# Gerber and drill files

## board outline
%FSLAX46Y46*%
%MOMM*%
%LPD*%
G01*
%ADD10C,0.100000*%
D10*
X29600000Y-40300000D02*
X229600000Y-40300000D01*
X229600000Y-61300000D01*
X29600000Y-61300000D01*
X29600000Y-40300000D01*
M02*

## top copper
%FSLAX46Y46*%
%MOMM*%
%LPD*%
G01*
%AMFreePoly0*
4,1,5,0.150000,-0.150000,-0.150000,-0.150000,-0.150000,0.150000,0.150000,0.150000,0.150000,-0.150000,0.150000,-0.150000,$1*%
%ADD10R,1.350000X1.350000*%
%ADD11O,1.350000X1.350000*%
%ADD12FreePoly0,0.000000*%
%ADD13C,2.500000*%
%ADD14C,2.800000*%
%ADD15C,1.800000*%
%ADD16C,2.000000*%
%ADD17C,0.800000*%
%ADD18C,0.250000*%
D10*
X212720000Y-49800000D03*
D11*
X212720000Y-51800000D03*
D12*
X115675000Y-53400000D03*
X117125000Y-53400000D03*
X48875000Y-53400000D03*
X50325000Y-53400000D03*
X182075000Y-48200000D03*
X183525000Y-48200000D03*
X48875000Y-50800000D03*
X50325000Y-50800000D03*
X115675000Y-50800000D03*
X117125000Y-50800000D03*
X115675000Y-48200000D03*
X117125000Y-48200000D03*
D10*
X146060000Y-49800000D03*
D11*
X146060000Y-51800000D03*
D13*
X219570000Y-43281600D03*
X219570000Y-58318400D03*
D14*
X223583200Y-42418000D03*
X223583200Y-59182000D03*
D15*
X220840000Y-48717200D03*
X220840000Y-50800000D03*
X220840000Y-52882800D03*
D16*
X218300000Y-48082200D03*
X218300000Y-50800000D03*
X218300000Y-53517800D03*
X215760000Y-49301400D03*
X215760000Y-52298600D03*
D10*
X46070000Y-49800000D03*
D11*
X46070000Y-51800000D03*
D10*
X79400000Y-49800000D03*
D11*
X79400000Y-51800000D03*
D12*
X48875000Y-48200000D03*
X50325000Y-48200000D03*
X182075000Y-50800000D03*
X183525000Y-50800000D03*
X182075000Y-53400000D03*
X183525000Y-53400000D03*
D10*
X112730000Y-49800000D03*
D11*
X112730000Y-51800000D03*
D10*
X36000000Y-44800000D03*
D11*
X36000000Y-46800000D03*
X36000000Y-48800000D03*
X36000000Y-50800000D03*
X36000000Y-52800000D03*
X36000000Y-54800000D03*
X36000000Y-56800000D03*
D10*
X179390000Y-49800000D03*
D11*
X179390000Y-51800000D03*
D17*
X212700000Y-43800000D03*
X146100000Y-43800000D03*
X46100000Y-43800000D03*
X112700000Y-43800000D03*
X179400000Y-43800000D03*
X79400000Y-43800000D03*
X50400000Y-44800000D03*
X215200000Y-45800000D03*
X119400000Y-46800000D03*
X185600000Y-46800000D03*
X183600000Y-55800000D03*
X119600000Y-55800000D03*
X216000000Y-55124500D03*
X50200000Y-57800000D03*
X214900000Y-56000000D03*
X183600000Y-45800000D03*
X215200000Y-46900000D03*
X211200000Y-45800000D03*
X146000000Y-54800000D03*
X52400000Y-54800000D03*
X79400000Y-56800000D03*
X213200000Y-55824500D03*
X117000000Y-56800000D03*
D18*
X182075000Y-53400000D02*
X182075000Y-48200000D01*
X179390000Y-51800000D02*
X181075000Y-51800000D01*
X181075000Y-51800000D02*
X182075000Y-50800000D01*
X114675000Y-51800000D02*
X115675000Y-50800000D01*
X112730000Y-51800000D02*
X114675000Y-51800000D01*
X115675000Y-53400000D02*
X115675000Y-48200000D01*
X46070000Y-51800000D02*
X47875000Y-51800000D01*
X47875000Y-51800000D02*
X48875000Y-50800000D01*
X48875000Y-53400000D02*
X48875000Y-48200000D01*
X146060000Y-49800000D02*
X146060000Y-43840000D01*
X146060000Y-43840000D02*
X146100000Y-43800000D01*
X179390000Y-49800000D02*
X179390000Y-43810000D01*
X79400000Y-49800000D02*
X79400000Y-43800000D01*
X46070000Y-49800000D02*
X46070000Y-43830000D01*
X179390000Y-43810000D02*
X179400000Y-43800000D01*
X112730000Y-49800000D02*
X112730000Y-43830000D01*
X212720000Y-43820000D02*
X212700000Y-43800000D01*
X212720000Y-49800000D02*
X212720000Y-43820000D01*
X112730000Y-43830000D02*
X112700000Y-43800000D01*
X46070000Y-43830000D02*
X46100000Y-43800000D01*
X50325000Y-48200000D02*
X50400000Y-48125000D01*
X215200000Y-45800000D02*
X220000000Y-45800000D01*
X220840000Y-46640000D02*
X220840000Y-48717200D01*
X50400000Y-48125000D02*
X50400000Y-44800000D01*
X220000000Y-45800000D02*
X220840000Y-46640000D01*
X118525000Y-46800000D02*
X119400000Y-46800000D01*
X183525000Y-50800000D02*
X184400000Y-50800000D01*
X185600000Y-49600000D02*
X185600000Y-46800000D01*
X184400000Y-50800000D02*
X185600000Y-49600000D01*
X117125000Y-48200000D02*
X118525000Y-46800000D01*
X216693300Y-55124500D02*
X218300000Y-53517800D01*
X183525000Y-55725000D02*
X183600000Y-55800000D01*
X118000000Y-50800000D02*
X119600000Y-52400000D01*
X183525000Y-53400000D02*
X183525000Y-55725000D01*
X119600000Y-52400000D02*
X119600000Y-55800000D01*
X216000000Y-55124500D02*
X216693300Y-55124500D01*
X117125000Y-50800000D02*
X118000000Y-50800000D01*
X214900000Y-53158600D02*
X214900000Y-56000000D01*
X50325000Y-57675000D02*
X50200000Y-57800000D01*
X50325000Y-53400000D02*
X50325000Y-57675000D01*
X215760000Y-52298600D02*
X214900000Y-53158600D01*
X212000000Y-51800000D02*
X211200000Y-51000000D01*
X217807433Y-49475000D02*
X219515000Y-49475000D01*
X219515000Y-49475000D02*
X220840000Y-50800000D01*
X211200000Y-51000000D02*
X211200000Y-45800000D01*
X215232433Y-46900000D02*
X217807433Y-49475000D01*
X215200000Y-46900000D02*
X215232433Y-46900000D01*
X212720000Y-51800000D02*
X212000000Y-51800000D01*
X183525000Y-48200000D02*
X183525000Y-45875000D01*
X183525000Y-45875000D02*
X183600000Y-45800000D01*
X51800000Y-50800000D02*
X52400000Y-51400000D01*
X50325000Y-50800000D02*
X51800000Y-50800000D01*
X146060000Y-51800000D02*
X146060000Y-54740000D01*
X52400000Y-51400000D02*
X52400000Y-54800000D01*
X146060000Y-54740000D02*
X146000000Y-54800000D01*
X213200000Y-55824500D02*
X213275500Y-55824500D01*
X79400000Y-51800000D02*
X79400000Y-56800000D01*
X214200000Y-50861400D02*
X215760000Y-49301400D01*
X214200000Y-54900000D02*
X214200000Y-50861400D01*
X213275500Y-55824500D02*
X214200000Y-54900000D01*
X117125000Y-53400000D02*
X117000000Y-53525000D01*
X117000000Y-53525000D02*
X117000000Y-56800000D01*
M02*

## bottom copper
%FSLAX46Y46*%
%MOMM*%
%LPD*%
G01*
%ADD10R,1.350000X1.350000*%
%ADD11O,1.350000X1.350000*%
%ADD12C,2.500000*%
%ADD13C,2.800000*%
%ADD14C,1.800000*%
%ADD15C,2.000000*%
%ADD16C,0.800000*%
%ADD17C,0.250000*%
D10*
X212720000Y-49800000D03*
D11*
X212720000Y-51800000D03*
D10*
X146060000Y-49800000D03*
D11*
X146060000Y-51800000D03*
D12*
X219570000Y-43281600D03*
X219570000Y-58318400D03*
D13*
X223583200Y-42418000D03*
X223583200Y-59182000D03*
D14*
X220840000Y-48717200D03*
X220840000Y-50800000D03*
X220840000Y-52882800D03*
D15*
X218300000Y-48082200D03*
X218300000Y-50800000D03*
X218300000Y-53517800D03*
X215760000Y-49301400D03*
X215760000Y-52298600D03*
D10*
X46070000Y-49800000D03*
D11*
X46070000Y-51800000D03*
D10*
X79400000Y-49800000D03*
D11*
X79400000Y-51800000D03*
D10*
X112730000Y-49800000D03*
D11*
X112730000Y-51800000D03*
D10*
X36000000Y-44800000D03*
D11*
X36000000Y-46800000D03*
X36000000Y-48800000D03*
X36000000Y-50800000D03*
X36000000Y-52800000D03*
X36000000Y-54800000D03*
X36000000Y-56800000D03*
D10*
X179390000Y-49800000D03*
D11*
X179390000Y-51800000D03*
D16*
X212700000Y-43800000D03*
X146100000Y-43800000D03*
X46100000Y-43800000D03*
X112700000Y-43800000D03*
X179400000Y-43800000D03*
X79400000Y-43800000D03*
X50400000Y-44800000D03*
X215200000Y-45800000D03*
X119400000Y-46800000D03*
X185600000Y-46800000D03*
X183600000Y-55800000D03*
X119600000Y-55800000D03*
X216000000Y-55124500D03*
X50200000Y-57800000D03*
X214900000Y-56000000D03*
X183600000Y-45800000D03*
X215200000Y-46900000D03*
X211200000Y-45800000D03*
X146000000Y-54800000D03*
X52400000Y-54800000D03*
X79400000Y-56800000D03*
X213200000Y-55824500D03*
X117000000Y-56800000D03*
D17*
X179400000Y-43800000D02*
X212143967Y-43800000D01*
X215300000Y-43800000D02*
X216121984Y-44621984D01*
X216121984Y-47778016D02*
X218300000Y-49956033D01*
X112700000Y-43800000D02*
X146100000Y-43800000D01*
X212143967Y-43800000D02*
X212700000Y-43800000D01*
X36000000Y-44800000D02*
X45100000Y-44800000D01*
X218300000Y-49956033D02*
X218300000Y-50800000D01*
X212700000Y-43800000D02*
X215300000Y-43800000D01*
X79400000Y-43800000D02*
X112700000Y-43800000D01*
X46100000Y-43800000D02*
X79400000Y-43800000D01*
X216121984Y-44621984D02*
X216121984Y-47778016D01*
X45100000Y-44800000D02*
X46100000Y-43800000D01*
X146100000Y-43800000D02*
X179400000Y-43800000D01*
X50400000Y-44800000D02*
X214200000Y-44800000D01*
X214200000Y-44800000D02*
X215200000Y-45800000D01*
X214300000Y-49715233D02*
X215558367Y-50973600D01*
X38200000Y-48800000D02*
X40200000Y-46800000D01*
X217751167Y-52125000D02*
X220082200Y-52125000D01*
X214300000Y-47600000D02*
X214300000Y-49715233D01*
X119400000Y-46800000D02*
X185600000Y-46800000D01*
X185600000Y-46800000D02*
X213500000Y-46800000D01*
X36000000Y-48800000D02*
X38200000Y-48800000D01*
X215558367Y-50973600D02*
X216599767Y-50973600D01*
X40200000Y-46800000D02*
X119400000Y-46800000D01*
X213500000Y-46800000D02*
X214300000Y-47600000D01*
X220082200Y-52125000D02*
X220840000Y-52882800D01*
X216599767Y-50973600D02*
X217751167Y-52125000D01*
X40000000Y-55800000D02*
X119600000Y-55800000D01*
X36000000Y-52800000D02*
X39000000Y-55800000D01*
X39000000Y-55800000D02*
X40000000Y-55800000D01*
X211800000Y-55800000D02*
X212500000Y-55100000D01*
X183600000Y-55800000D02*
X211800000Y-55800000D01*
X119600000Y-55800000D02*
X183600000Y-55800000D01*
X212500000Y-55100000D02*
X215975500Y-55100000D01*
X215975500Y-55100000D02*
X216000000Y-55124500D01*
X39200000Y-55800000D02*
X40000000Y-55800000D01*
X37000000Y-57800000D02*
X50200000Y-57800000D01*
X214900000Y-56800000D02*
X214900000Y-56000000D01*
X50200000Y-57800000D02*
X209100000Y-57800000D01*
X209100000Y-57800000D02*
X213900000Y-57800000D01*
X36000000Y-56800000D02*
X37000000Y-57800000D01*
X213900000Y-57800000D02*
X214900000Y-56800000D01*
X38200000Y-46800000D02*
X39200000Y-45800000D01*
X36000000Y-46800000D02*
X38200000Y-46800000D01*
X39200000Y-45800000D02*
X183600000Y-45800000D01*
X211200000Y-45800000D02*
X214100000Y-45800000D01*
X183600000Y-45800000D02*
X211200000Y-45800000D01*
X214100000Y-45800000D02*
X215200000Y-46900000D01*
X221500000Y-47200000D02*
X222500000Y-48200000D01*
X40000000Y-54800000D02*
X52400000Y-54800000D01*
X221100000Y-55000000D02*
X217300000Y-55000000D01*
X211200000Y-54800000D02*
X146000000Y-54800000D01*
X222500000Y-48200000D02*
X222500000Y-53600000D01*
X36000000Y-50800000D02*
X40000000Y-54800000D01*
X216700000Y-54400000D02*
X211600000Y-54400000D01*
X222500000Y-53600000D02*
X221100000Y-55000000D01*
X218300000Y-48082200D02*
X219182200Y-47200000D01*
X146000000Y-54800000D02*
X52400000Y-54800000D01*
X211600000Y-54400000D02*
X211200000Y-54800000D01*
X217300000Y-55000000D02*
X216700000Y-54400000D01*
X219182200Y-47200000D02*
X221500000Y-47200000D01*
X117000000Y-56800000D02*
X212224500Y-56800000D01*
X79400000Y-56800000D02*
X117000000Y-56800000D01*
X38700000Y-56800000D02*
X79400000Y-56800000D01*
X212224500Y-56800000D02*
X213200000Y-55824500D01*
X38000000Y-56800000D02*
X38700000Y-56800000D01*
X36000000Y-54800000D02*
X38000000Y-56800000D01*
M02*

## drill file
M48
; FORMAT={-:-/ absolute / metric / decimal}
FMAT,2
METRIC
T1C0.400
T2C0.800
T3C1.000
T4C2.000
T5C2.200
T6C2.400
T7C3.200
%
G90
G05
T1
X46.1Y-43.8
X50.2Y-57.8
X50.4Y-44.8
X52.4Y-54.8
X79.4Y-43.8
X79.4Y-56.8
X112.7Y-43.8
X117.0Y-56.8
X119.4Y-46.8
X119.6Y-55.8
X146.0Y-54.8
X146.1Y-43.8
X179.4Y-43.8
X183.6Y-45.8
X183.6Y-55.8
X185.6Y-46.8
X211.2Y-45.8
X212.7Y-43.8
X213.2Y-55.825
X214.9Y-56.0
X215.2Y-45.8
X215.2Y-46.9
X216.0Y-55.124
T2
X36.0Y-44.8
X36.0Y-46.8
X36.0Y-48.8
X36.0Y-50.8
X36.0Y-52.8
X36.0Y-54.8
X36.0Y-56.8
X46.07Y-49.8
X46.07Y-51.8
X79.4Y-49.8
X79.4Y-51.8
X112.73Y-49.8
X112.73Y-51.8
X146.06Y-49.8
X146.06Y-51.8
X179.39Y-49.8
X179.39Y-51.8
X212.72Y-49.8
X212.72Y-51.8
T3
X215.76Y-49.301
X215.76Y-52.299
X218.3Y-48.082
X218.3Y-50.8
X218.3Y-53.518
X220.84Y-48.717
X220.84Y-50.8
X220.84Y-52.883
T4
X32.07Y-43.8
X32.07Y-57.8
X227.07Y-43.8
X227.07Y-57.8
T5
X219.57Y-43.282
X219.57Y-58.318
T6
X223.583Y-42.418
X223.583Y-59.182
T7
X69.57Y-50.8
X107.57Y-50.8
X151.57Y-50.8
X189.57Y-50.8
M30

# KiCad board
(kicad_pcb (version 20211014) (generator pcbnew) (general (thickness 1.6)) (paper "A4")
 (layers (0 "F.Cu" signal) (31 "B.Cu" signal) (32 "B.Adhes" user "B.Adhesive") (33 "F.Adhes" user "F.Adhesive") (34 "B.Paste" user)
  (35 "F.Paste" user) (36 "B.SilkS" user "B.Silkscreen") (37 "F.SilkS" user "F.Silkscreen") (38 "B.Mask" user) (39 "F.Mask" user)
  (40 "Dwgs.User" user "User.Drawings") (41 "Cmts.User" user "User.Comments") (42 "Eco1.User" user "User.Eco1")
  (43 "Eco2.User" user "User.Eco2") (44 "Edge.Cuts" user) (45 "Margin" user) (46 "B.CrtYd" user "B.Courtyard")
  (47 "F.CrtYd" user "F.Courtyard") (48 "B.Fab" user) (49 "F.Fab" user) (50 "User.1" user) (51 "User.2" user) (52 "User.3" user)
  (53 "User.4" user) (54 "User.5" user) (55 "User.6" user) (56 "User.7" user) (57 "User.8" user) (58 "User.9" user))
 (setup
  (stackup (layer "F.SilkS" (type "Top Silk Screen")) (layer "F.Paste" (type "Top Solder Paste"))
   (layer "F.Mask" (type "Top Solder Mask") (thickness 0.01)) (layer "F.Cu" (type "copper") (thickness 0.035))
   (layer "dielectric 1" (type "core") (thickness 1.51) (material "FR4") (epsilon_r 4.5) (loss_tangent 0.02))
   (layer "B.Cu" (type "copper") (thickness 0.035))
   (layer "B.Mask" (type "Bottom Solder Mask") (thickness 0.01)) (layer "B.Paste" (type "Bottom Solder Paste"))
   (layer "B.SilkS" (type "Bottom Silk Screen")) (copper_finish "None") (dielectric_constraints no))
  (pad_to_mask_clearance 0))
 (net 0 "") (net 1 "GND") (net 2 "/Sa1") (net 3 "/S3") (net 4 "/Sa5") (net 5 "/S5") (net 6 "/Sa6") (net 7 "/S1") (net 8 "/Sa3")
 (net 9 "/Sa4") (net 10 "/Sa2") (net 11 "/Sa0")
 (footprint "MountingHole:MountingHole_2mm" (layer "F.Cu") (at 32.07 57.8)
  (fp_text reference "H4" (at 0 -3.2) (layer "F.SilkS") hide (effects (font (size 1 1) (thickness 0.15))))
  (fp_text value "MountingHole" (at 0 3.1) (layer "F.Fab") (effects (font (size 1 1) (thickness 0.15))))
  (pad "" np_thru_hole circle (at 0 0) (size 2 2) (drill 2) (layers *.Cu *.Mask)))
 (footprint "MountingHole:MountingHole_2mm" (layer "F.Cu") (at 227.07 57.8)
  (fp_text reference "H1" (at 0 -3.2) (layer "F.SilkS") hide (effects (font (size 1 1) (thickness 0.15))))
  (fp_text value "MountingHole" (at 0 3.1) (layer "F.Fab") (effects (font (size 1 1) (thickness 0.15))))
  (pad "" np_thru_hole circle (at 0 0) (size 2 2) (drill 2) (layers *.Cu *.Mask)))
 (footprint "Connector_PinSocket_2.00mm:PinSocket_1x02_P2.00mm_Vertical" (layer "F.Cu") (at 212.72 49.8)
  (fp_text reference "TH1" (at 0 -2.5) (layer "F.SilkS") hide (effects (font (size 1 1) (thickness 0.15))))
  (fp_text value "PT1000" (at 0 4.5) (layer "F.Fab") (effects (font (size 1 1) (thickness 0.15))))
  (pad "1" thru_hole rect (at 0 0) (size 1.35 1.35) (drill 0.8) (layers *.Cu *.Mask) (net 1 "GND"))
  (pad "2" thru_hole oval (at 0 2) (size 1.35 1.35) (drill 0.8) (layers *.Cu *.Mask) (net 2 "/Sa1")))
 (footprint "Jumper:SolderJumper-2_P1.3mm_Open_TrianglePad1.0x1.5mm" (layer "F.Cu") (at 116.4 53.4)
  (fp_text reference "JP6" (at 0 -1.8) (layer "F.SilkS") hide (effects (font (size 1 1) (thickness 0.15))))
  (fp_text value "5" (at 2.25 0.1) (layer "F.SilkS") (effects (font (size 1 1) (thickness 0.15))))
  (pad "1" smd custom (at -0.725 0) (size 0.3 0.3) (layers "F.Cu" "F.Mask") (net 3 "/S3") (zone_connect 2)
   (options (clearance outline) (anchor rect)) (primitives))
  (pad "2" smd custom (at 0.725 0) (size 0.3 0.3) (layers "F.Cu" "F.Mask") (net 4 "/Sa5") (zone_connect 2)
   (options (clearance outline) (anchor rect)) (primitives)))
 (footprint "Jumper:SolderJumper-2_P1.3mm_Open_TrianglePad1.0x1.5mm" (layer "F.Cu") (at 49.6 53.4)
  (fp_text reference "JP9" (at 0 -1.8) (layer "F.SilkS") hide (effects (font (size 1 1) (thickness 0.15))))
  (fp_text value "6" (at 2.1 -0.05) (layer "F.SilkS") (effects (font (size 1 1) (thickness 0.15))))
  (pad "1" smd custom (at -0.725 0) (size 0.3 0.3) (layers "F.Cu" "F.Mask") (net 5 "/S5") (zone_connect 2)
   (options (clearance outline) (anchor rect)) (primitives))
  (pad "2" smd custom (at 0.725 0) (size 0.3 0.3) (layers "F.Cu" "F.Mask") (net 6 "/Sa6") (zone_connect 2)
   (options (clearance outline) (anchor rect)) (primitives)))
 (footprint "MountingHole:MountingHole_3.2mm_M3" (layer "F.Cu") (at 69.57 50.8)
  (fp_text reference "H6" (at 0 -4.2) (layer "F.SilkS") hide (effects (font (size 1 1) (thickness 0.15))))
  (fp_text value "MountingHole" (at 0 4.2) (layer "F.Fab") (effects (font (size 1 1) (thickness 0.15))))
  (pad "" np_thru_hole circle (at 0 0) (size 3.2 3.2) (drill 3.2) (layers *.Cu *.Mask)))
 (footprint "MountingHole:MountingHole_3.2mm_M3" (layer "F.Cu") (at 107.57 50.8)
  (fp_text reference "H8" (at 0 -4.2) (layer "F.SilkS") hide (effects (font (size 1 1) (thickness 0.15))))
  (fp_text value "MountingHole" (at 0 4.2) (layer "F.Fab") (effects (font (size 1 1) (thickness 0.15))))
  (pad "" np_thru_hole circle (at 0 0) (size 3.2 3.2) (drill 3.2) (layers *.Cu *.Mask)))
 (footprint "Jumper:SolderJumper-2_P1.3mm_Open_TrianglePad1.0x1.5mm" (layer "F.Cu") (at 182.8 48.2)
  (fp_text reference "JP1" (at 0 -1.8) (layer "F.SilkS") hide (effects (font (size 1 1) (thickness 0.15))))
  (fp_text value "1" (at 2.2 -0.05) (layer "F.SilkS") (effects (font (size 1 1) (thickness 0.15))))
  (pad "1" smd custom (at -0.725 0) (size 0.3 0.3) (layers "F.Cu" "F.Mask") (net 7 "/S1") (zone_connect 2)
   (options (clearance outline) (anchor rect)) (primitives))
  (pad "2" smd custom (at 0.725 0) (size 0.3 0.3) (layers "F.Cu" "F.Mask") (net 2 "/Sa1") (zone_connect 2)
   (options (clearance outline) (anchor rect)) (primitives)))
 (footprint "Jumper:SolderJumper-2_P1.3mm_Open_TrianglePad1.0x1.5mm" (layer "F.Cu") (at 49.6 50.8)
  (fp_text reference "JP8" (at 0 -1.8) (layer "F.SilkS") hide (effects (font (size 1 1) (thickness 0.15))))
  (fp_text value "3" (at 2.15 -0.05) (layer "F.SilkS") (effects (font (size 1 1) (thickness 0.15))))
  (pad "1" smd custom (at -0.725 0) (size 0.3 0.3) (layers "F.Cu" "F.Mask") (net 5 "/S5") (zone_connect 2)
   (options (clearance outline) (anchor rect)) (primitives))
  (pad "2" smd custom (at 0.725 0) (size 0.3 0.3) (layers "F.Cu" "F.Mask") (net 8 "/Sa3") (zone_connect 2)
   (options (clearance outline) (anchor rect)) (primitives)))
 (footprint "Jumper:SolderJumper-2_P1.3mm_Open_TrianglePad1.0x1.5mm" (layer "F.Cu") (at 116.4 50.8)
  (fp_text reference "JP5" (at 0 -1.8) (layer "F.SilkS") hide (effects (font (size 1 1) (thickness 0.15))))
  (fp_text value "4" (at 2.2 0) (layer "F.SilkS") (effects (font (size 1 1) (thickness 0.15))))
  (pad "1" smd custom (at -0.725 0) (size 0.3 0.3) (layers "F.Cu" "F.Mask") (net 3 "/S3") (zone_connect 2)
   (options (clearance outline) (anchor rect)) (primitives))
  (pad "2" smd custom (at 0.725 0) (size 0.3 0.3) (layers "F.Cu" "F.Mask") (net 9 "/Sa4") (zone_connect 2)
   (options (clearance outline) (anchor rect)) (primitives)))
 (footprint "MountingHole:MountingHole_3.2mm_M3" (layer "F.Cu") (at 151.57 50.8)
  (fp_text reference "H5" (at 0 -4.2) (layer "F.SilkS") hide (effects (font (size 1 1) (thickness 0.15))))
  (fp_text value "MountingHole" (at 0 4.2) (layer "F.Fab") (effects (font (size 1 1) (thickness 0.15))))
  (pad "" np_thru_hole circle (at 0 0) (size 3.2 3.2) (drill 3.2) (layers *.Cu *.Mask)))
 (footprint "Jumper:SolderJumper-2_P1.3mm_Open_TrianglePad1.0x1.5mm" (layer "F.Cu") (at 116.4 48.2)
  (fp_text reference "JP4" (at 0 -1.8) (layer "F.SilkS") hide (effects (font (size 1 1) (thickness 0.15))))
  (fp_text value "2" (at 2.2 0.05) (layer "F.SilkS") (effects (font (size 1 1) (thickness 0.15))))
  (pad "1" smd custom (at -0.725 0) (size 0.3 0.3) (layers "F.Cu" "F.Mask") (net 3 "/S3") (zone_connect 2)
   (options (clearance outline) (anchor rect)) (primitives))
  (pad "2" smd custom (at 0.725 0) (size 0.3 0.3) (layers "F.Cu" "F.Mask") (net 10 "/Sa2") (zone_connect 2)
   (options (clearance outline) (anchor rect)) (primitives)))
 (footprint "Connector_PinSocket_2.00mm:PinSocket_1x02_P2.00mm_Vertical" (layer "F.Cu") (at 146.06 49.8)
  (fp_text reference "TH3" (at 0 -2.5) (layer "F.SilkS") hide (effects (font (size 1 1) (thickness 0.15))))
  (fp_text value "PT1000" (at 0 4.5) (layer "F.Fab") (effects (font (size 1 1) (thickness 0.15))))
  (pad "1" thru_hole rect (at 0 0) (size 1.35 1.35) (drill 0.8) (layers *.Cu *.Mask) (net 1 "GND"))
  (pad "2" thru_hole oval (at 0 2) (size 1.35 1.35) (drill 0.8) (layers *.Cu *.Mask) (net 8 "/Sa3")))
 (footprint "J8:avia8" (layer "F.Cu") (at 218.3 50.8 -90)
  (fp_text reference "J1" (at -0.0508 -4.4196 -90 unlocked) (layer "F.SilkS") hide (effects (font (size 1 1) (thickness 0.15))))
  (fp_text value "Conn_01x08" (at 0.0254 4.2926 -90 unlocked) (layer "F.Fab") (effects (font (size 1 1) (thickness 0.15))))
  (pad "" np_thru_hole circle (at -7.5184 -1.27 270) (size 2.5 2.5) (drill 2.2) (layers F&B.Cu *.Mask))
  (pad "" np_thru_hole circle (at 7.5184 -1.27 270) (size 2.5 2.5) (drill 2.2) (layers F&B.Cu *.Mask))
  (pad "" np_thru_hole circle (at -8.382 -5.2832 270) (size 2.8 2.8) (drill 2.4) (layers F&B.Cu *.Mask))
  (pad "" np_thru_hole circle (at 8.382 -5.2832 270) (size 2.8 2.8) (drill 2.4) (layers F&B.Cu *.Mask))
  (pad "1" thru_hole circle (at -2.0828 -2.54 270) (size 1.8 1.8) (drill 1) (layers *.Cu *.Mask) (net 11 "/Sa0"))
  (pad "2" thru_hole circle (at 0 -2.54 270) (size 1.8 1.8) (drill 1) (layers *.Cu *.Mask) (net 2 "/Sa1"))
  (pad "3" thru_hole circle (at 2.0828 -2.54 270) (size 1.8 1.8) (drill 1) (layers *.Cu *.Mask) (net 10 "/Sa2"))
  (pad "4" thru_hole circle (at -2.7178 0 270) (size 2 2) (drill 1) (layers *.Cu *.Mask) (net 8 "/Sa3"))
  (pad "5" thru_hole circle (at 0 0 270) (size 2 2) (drill 1) (layers *.Cu *.Mask) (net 1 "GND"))
  (pad "6" thru_hole circle (at 2.7178 0 270) (size 2 2) (drill 1) (layers *.Cu *.Mask) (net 9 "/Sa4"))
  (pad "7" thru_hole circle (at -1.4986 2.54 270) (size 2 2) (drill 1) (layers *.Cu *.Mask) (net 4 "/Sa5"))
  (pad "8" thru_hole circle (at 1.4986 2.54 270) (size 2 2) (drill 1) (layers *.Cu *.Mask) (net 6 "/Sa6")))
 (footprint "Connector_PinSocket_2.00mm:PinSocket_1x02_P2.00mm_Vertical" (layer "F.Cu") (at 46.07 49.8)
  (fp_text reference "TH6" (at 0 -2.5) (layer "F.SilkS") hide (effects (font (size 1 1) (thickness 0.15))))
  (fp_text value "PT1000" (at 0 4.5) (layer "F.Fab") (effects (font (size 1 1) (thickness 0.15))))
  (pad "1" thru_hole rect (at 0 0) (size 1.35 1.35) (drill 0.8) (layers *.Cu *.Mask) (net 1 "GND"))
  (pad "2" thru_hole oval (at 0 2) (size 1.35 1.35) (drill 0.8) (layers *.Cu *.Mask) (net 5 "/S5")))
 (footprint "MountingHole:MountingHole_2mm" (layer "F.Cu") (at 227.07 43.8)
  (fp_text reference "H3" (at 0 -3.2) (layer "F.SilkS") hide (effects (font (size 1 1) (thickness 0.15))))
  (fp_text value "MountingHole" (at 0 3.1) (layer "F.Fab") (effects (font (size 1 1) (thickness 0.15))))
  (pad "" np_thru_hole circle (at 0 0) (size 2 2) (drill 2) (layers *.Cu *.Mask)))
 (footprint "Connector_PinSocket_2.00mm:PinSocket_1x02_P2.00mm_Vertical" (layer "F.Cu") (at 79.4 49.8)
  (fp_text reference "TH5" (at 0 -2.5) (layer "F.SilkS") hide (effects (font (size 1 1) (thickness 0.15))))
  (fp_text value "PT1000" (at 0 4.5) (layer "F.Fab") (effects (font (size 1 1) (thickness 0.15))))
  (pad "1" thru_hole rect (at 0 0) (size 1.35 1.35) (drill 0.8) (layers *.Cu *.Mask) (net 1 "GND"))
  (pad "2" thru_hole oval (at 0 2) (size 1.35 1.35) (drill 0.8) (layers *.Cu *.Mask) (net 4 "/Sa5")))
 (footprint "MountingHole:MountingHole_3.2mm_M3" (layer "F.Cu") (at 189.57 50.8)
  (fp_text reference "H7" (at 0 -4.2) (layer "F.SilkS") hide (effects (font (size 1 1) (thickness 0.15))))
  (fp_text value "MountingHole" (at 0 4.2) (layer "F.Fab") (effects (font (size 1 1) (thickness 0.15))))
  (pad "" np_thru_hole circle (at 0 0) (size 3.2 3.2) (drill 3.2) (layers *.Cu *.Mask)))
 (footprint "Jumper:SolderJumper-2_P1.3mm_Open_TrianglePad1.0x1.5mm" (layer "F.Cu") (at 49.6 48.2)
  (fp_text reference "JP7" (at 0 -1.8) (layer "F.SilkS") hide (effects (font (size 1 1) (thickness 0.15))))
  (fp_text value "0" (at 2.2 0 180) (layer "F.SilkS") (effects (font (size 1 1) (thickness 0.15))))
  (pad "1" smd custom (at -0.725 0) (size 0.3 0.3) (layers "F.Cu" "F.Mask") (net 5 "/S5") (zone_connect 2)
   (options (clearance outline) (anchor rect)) (primitives))
  (pad "2" smd custom (at 0.725 0) (size 0.3 0.3) (layers "F.Cu" "F.Mask") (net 11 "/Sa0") (zone_connect 2)
   (options (clearance outline) (anchor rect)) (primitives)))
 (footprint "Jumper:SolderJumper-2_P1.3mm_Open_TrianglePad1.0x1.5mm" (layer "F.Cu") (at 182.8 50.8)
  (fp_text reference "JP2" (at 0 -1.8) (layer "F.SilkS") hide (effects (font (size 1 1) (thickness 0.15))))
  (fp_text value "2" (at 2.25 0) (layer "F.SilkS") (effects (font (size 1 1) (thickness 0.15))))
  (pad "1" smd custom (at -0.725 0) (size 0.3 0.3) (layers "F.Cu" "F.Mask") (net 7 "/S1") (zone_connect 2)
   (options (clearance outline) (anchor rect)) (primitives))
  (pad "2" smd custom (at 0.725 0) (size 0.3 0.3) (layers "F.Cu" "F.Mask") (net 10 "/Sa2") (zone_connect 2)
   (options (clearance outline) (anchor rect)) (primitives)))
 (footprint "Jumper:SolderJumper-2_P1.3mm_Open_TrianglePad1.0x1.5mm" (layer "F.Cu") (at 182.8 53.4)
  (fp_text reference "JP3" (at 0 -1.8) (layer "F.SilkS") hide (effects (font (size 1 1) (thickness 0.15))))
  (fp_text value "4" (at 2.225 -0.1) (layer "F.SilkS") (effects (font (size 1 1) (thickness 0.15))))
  (pad "1" smd custom (at -0.725 0) (size 0.3 0.3) (layers "F.Cu" "F.Mask") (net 7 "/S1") (zone_connect 2)
   (options (clearance outline) (anchor rect)) (primitives))
  (pad "2" smd custom (at 0.725 0) (size 0.3 0.3) (layers "F.Cu" "F.Mask") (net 9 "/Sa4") (zone_connect 2)
   (options (clearance outline) (anchor rect)) (primitives)))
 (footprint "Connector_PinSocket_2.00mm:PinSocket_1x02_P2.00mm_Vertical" (layer "F.Cu") (at 112.73 49.8)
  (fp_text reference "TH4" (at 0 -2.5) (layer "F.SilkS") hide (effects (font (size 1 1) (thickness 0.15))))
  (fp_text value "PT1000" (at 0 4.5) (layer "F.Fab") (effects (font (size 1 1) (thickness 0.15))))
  (pad "1" thru_hole rect (at 0 0) (size 1.35 1.35) (drill 0.8) (layers *.Cu *.Mask) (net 1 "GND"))
  (pad "2" thru_hole oval (at 0 2) (size 1.35 1.35) (drill 0.8) (layers *.Cu *.Mask) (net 3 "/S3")))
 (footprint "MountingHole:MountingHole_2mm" (layer "F.Cu") (at 32.07 43.8)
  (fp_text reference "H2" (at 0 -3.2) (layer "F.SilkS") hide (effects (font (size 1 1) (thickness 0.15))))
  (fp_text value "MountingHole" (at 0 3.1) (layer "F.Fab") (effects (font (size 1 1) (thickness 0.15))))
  (pad "" np_thru_hole circle (at 0 0) (size 2 2) (drill 2) (layers *.Cu *.Mask)))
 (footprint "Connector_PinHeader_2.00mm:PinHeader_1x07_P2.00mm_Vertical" (layer "F.Cu") (at 36 44.8)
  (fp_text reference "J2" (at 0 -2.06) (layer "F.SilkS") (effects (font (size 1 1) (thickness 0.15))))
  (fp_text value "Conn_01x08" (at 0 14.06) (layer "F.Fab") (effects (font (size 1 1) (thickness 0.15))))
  (pad "1" thru_hole rect (at 0 0) (size 1.35 1.35) (drill 0.8) (layers *.Cu *.Mask) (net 1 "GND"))
  (pad "2" thru_hole oval (at 0 2) (size 1.35 1.35) (drill 0.8) (layers *.Cu *.Mask) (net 2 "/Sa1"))
  (pad "3" thru_hole oval (at 0 4) (size 1.35 1.35) (drill 0.8) (layers *.Cu *.Mask) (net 10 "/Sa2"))
  (pad "4" thru_hole oval (at 0 6) (size 1.35 1.35) (drill 0.8) (layers *.Cu *.Mask) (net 8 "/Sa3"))
  (pad "5" thru_hole oval (at 0 8) (size 1.35 1.35) (drill 0.8) (layers *.Cu *.Mask) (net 9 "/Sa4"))
  (pad "6" thru_hole oval (at 0 10) (size 1.35 1.35) (drill 0.8) (layers *.Cu *.Mask) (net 4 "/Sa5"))
  (pad "7" thru_hole oval (at 0 12) (size 1.35 1.35) (drill 0.8) (layers *.Cu *.Mask) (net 6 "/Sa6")))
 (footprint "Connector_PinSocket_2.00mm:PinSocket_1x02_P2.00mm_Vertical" (layer "F.Cu") (at 179.39 49.8)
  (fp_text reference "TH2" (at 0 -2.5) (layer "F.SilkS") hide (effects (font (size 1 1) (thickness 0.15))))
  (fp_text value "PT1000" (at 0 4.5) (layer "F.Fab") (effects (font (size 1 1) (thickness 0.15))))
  (pad "1" thru_hole rect (at 0 0) (size 1.35 1.35) (drill 0.8) (layers *.Cu *.Mask) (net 1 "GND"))
  (pad "2" thru_hole oval (at 0 2) (size 1.35 1.35) (drill 0.8) (layers *.Cu *.Mask) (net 7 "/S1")))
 (gr_rect (start 29.6 40.3) (end 229.6 61.3) (layer "Edge.Cuts") (width 0.1) (fill none))
 (segment (start 182.075 53.4) (end 182.075 48.2) (width 0.25) (layer "F.Cu") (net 7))
 (segment (start 179.39 51.8) (end 181.075 51.8) (width 0.25) (layer "F.Cu") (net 7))
 (segment (start 181.075 51.8) (end 182.075 50.8) (width 0.25) (layer "F.Cu") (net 7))
 (segment (start 114.675 51.8) (end 115.675 50.8) (width 0.25) (layer "F.Cu") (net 3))
 (segment (start 112.73 51.8) (end 114.675 51.8) (width 0.25) (layer "F.Cu") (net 3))
 (segment (start 115.675 53.4) (end 115.675 48.2) (width 0.25) (layer "F.Cu") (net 3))
 (segment (start 46.07 51.8) (end 47.875 51.8) (width 0.25) (layer "F.Cu") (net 5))
 (segment (start 47.875 51.8) (end 48.875 50.8) (width 0.25) (layer "F.Cu") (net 5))
 (segment (start 48.875 53.4) (end 48.875 48.2) (width 0.25) (layer "F.Cu") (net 5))
 (segment (start 146.06 49.8) (end 146.06 43.84) (width 0.25) (layer "F.Cu") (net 1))
 (segment (start 146.06 43.84) (end 146.1 43.8) (width 0.25) (layer "F.Cu") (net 1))
 (segment (start 179.39 49.8) (end 179.39 43.81) (width 0.25) (layer "F.Cu") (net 1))
 (segment (start 79.4 49.8) (end 79.4 43.8) (width 0.25) (layer "F.Cu") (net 1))
 (segment (start 46.07 49.8) (end 46.07 43.83) (width 0.25) (layer "F.Cu") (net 1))
 (segment (start 179.39 43.81) (end 179.4 43.8) (width 0.25) (layer "F.Cu") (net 1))
 (segment (start 112.73 49.8) (end 112.73 43.83) (width 0.25) (layer "F.Cu") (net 1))
 (segment (start 212.72 43.82) (end 212.7 43.8) (width 0.25) (layer "F.Cu") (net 1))
 (segment (start 212.72 49.8) (end 212.72 43.82) (width 0.25) (layer "F.Cu") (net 1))
 (segment (start 112.73 43.83) (end 112.7 43.8) (width 0.25) (layer "F.Cu") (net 1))
 (segment (start 46.07 43.83) (end 46.1 43.8) (width 0.25) (layer "F.Cu") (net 1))
 (via (at 212.7 43.8) (size 0.8) (drill 0.4) (layers "F.Cu" "B.Cu") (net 1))
 (via (at 146.1 43.8) (size 0.8) (drill 0.4) (layers "F.Cu" "B.Cu") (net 1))
 (via (at 46.1 43.8) (size 0.8) (drill 0.4) (layers "F.Cu" "B.Cu") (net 1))
 (via (at 112.7 43.8) (size 0.8) (drill 0.4) (layers "F.Cu" "B.Cu") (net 1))
 (via (at 179.4 43.8) (size 0.8) (drill 0.4) (layers "F.Cu" "B.Cu") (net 1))
 (via (at 79.4 43.8) (size 0.8) (drill 0.4) (layers "F.Cu" "B.Cu") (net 1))
 (segment (start 179.4 43.8) (end 212.143967 43.8) (width 0.25) (layer "B.Cu") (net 1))
 (segment (start 215.3 43.8) (end 216.121984 44.621984) (width 0.25) (layer "B.Cu") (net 1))
 (segment (start 216.121984 47.778016) (end 218.3 49.956033) (width 0.25) (layer "B.Cu") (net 1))
 (segment (start 112.7 43.8) (end 146.1 43.8) (width 0.25) (layer "B.Cu") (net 1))
 (segment (start 212.143967 43.8) (end 212.7 43.8) (width 0.25) (layer "B.Cu") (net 1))
 (segment (start 36 44.8) (end 45.1 44.8) (width 0.25) (layer "B.Cu") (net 1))
 (segment (start 218.3 49.956033) (end 218.3 50.8) (width 0.25) (layer "B.Cu") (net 1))
 (segment (start 212.7 43.8) (end 215.3 43.8) (width 0.25) (layer "B.Cu") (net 1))
 (segment (start 79.4 43.8) (end 112.7 43.8) (width 0.25) (layer "B.Cu") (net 1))
 (segment (start 46.1 43.8) (end 79.4 43.8) (width 0.25) (layer "B.Cu") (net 1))
 (segment (start 216.121984 44.621984) (end 216.121984 47.778016) (width 0.25) (layer "B.Cu") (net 1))
 (segment (start 45.1 44.8) (end 46.1 43.8) (width 0.25) (layer "B.Cu") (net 1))
 (segment (start 146.1 43.8) (end 179.4 43.8) (width 0.25) (layer "B.Cu") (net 1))
 (segment (start 50.325 48.2) (end 50.4 48.125) (width 0.25) (layer "F.Cu") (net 11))
 (segment (start 215.2 45.8) (end 220 45.8) (width 0.25) (layer "F.Cu") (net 11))
 (segment (start 220.84 46.64) (end 220.84 48.7172) (width 0.25) (layer "F.Cu") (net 11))
 (segment (start 50.4 48.125) (end 50.4 44.8) (width 0.25) (layer "F.Cu") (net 11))
 (segment (start 220 45.8) (end 220.84 46.64) (width 0.25) (layer "F.Cu") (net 11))
 (via (at 50.4 44.8) (size 0.8) (drill 0.4) (layers "F.Cu" "B.Cu") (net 11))
 (via (at 215.2 45.8) (size 0.8) (drill 0.4) (layers "F.Cu" "B.Cu") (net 11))
 (segment (start 50.4 44.8) (end 214.2 44.8) (width 0.25) (layer "B.Cu") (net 11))
 (segment (start 214.2 44.8) (end 215.2 45.8) (width 0.25) (layer "B.Cu") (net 11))
 (segment (start 118.525 46.8) (end 119.4 46.8) (width 0.25) (layer "F.Cu") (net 10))
 (segment (start 183.525 50.8) (end 184.4 50.8) (width 0.25) (layer "F.Cu") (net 10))
 (segment (start 185.6 49.6) (end 185.6 46.8) (width 0.25) (layer "F.Cu") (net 10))
 (segment (start 184.4 50.8) (end 185.6 49.6) (width 0.25) (layer "F.Cu") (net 10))
 (segment (start 117.125 48.2) (end 118.525 46.8) (width 0.25) (layer "F.Cu") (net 10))
 (via (at 119.4 46.8) (size 0.8) (drill 0.4) (layers "F.Cu" "B.Cu") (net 10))
 (via (at 185.6 46.8) (size 0.8) (drill 0.4) (layers "F.Cu" "B.Cu") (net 10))
 (segment (start 214.3 49.715233) (end 215.558367 50.9736) (width 0.25) (layer "B.Cu") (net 10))
 (segment (start 38.2 48.8) (end 40.2 46.8) (width 0.25) (layer "B.Cu") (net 10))
 (segment (start 217.751167 52.125) (end 220.0822 52.125) (width 0.25) (layer "B.Cu") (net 10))
 (segment (start 214.3 47.6) (end 214.3 49.715233) (width 0.25) (layer "B.Cu") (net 10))
 (segment (start 119.4 46.8) (end 185.6 46.8) (width 0.25) (layer "B.Cu") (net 10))
 (segment (start 185.6 46.8) (end 213.5 46.8) (width 0.25) (layer "B.Cu") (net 10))
 (segment (start 36 48.8) (end 38.2 48.8) (width 0.25) (layer "B.Cu") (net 10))
 (segment (start 215.558367 50.9736) (end 216.599767 50.9736) (width 0.25) (layer "B.Cu") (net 10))
 (segment (start 40.2 46.8) (end 119.4 46.8) (width 0.25) (layer "B.Cu") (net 10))
 (segment (start 213.5 46.8) (end 214.3 47.6) (width 0.25) (layer "B.Cu") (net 10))
 (segment (start 220.0822 52.125) (end 220.84 52.8828) (width 0.25) (layer "B.Cu") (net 10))
 (segment (start 216.599767 50.9736) (end 217.751167 52.125) (width 0.25) (layer "B.Cu") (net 10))
 (segment (start 216.6933 55.1245) (end 218.3 53.5178) (width 0.25) (layer "F.Cu") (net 9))
 (segment (start 183.525 55.725) (end 183.6 55.8) (width 0.25) (layer "F.Cu") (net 9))
 (segment (start 118 50.8) (end 119.6 52.4) (width 0.25) (layer "F.Cu") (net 9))
 (segment (start 183.525 53.4) (end 183.525 55.725) (width 0.25) (layer "F.Cu") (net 9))
 (segment (start 119.6 52.4) (end 119.6 55.8) (width 0.25) (layer "F.Cu") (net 9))
 (segment (start 216 55.1245) (end 216.6933 55.1245) (width 0.25) (layer "F.Cu") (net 9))
 (segment (start 117.125 50.8) (end 118 50.8) (width 0.25) (layer "F.Cu") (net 9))
 (via (at 183.6 55.8) (size 0.8) (drill 0.4) (layers "F.Cu" "B.Cu") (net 9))
 (via (at 119.6 55.8) (size 0.8) (drill 0.4) (layers "F.Cu" "B.Cu") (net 9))
 (via (at 216 55.1245) (size 0.8) (drill 0.4) (layers "F.Cu" "B.Cu") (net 9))
 (segment (start 40 55.8) (end 119.6 55.8) (width 0.25) (layer "B.Cu") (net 9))
 (segment (start 36 52.8) (end 39 55.8) (width 0.25) (layer "B.Cu") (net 9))
 (segment (start 39 55.8) (end 40 55.8) (width 0.25) (layer "B.Cu") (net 9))
 (segment (start 211.8 55.8) (end 212.5 55.1) (width 0.25) (layer "B.Cu") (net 9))
 (segment (start 183.6 55.8) (end 211.8 55.8) (width 0.25) (layer "B.Cu") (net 9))
 (segment (start 119.6 55.8) (end 183.6 55.8) (width 0.25) (layer "B.Cu") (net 9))
 (segment (start 212.5 55.1) (end 215.9755 55.1) (width 0.25) (layer "B.Cu") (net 9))
 (segment (start 215.9755 55.1) (end 216 55.1245) (width 0.25) (layer "B.Cu") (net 9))
 (segment (start 39.2 55.8) (end 40 55.8) (width 0.25) (layer "B.Cu") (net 9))
 (segment (start 214.9 53.1586) (end 214.9 56) (width 0.25) (layer "F.Cu") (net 6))
 (segment (start 50.325 57.675) (end 50.2 57.8) (width 0.25) (layer "F.Cu") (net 6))
 (segment (start 50.325 53.4) (end 50.325 57.675) (width 0.25) (layer "F.Cu") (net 6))
 (segment (start 215.76 52.2986) (end 214.9 53.1586) (width 0.25) (layer "F.Cu") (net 6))
 (via (at 50.2 57.8) (size 0.8) (drill 0.4) (layers "F.Cu" "B.Cu") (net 6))
 (via (at 214.9 56) (size 0.8) (drill 0.4) (layers "F.Cu" "B.Cu") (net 6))
 (segment (start 37 57.8) (end 50.2 57.8) (width 0.25) (layer "B.Cu") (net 6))
 (segment (start 214.9 56.8) (end 214.9 56) (width 0.25) (layer "B.Cu") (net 6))
 (segment (start 50.2 57.8) (end 209.1 57.8) (width 0.25) (layer "B.Cu") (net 6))
 (segment (start 209.1 57.8) (end 213.9 57.8) (width 0.25) (layer "B.Cu") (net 6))
 (segment (start 36 56.8) (end 37 57.8) (width 0.25) (layer "B.Cu") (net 6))
 (segment (start 213.9 57.8) (end 214.9 56.8) (width 0.25) (layer "B.Cu") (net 6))
 (segment (start 212 51.8) (end 211.2 51) (width 0.25) (layer "F.Cu") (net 2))
 (segment (start 217.807433 49.475) (end 219.515 49.475) (width 0.25) (layer "F.Cu") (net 2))
 (segment (start 219.515 49.475) (end 220.84 50.8) (width 0.25) (layer "F.Cu") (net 2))
 (segment (start 211.2 51) (end 211.2 45.8) (width 0.25) (layer "F.Cu") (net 2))
 (segment (start 215.232433 46.9) (end 217.807433 49.475) (width 0.25) (layer "F.Cu") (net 2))
 (segment (start 215.2 46.9) (end 215.232433 46.9) (width 0.25) (layer "F.Cu") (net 2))
 (segment (start 212.72 51.8) (end 212 51.8) (width 0.25) (layer "F.Cu") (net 2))
 (segment (start 183.525 48.2) (end 183.525 45.875) (width 0.25) (layer "F.Cu") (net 2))
 (segment (start 183.525 45.875) (end 183.6 45.8) (width 0.25) (layer "F.Cu") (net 2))
 (via (at 183.6 45.8) (size 0.8) (drill 0.4) (layers "F.Cu" "B.Cu") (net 2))
 (via (at 215.2 46.9) (size 0.8) (drill 0.4) (layers "F.Cu" "B.Cu") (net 2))
 (via (at 211.2 45.8) (size 0.8) (drill 0.4) (layers "F.Cu" "B.Cu") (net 2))
 (segment (start 38.2 46.8) (end 39.2 45.8) (width 0.25) (layer "B.Cu") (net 2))
 (segment (start 36 46.8) (end 38.2 46.8) (width 0.25) (layer "B.Cu") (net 2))
 (segment (start 39.2 45.8) (end 183.6 45.8) (width 0.25) (layer "B.Cu") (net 2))
 (segment (start 211.2 45.8) (end 214.1 45.8) (width 0.25) (layer "B.Cu") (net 2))
 (segment (start 183.6 45.8) (end 211.2 45.8) (width 0.25) (layer "B.Cu") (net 2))
 (segment (start 214.1 45.8) (end 215.2 46.9) (width 0.25) (layer "B.Cu") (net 2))
 (segment (start 51.8 50.8) (end 52.4 51.4) (width 0.25) (layer "F.Cu") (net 8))
 (segment (start 50.325 50.8) (end 51.8 50.8) (width 0.25) (layer "F.Cu") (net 8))
 (segment (start 146.06 51.8) (end 146.06 54.74) (width 0.25) (layer "F.Cu") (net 8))
 (segment (start 52.4 51.4) (end 52.4 54.8) (width 0.25) (layer "F.Cu") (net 8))
 (segment (start 146.06 54.74) (end 146 54.8) (width 0.25) (layer "F.Cu") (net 8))
 (via (at 146 54.8) (size 0.8) (drill 0.4) (layers "F.Cu" "B.Cu") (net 8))
 (via (at 52.4 54.8) (size 0.8) (drill 0.4) (layers "F.Cu" "B.Cu") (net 8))
 (segment (start 221.5 47.2) (end 222.5 48.2) (width 0.25) (layer "B.Cu") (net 8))
 (segment (start 40 54.8) (end 52.4 54.8) (width 0.25) (layer "B.Cu") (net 8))
 (segment (start 221.1 55) (end 217.3 55) (width 0.25) (layer "B.Cu") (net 8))
 (segment (start 211.2 54.8) (end 146 54.8) (width 0.25) (layer "B.Cu") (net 8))
 (segment (start 222.5 48.2) (end 222.5 53.6) (width 0.25) (layer "B.Cu") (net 8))
 (segment (start 36 50.8) (end 40 54.8) (width 0.25) (layer "B.Cu") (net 8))
 (segment (start 216.7 54.4) (end 211.6 54.4) (width 0.25) (layer "B.Cu") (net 8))
 (segment (start 222.5 53.6) (end 221.1 55) (width 0.25) (layer "B.Cu") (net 8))
 (segment (start 218.3 48.0822) (end 219.1822 47.2) (width 0.25) (layer "B.Cu") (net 8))
 (segment (start 146 54.8) (end 52.4 54.8) (width 0.25) (layer "B.Cu") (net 8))
 (segment (start 211.6 54.4) (end 211.2 54.8) (width 0.25) (layer "B.Cu") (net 8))
 (segment (start 217.3 55) (end 216.7 54.4) (width 0.25) (layer "B.Cu") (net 8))
 (segment (start 219.1822 47.2) (end 221.5 47.2) (width 0.25) (layer "B.Cu") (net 8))
 (segment (start 213.2 55.8245) (end 213.2755 55.8245) (width 0.25) (layer "F.Cu") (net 4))
 (segment (start 79.4 51.8) (end 79.4 56.8) (width 0.25) (layer "F.Cu") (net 4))
 (segment (start 214.2 50.8614) (end 215.76 49.3014) (width 0.25) (layer "F.Cu") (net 4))
 (segment (start 214.2 54.9) (end 214.2 50.8614) (width 0.25) (layer "F.Cu") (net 4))
 (segment (start 213.2755 55.8245) (end 214.2 54.9) (width 0.25) (layer "F.Cu") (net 4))
 (segment (start 117.125 53.4) (end 117 53.525) (width 0.25) (layer "F.Cu") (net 4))
 (segment (start 117 53.525) (end 117 56.8) (width 0.25) (layer "F.Cu") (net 4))
 (via (at 79.4 56.8) (size 0.8) (drill 0.4) (layers "F.Cu" "B.Cu") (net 4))
 (via (at 213.2 55.8245) (size 0.8) (drill 0.4) (layers "F.Cu" "B.Cu") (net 4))
 (via (at 117 56.8) (size 0.8) (drill 0.4) (layers "F.Cu" "B.Cu") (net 4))
 (segment (start 117 56.8) (end 212.2245 56.8) (width 0.25) (layer "B.Cu") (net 4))
 (segment (start 79.4 56.8) (end 117 56.8) (width 0.25) (layer "B.Cu") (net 4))
 (segment (start 38.7 56.8) (end 79.4 56.8) (width 0.25) (layer "B.Cu") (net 4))
 (segment (start 212.2245 56.8) (end 213.2 55.8245) (width 0.25) (layer "B.Cu") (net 4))
 (segment (start 38 56.8) (end 38.7 56.8) (width 0.25) (layer "B.Cu") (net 4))
 (segment (start 36 54.8) (end 38 56.8) (width 0.25) (layer "B.Cu") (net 4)))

